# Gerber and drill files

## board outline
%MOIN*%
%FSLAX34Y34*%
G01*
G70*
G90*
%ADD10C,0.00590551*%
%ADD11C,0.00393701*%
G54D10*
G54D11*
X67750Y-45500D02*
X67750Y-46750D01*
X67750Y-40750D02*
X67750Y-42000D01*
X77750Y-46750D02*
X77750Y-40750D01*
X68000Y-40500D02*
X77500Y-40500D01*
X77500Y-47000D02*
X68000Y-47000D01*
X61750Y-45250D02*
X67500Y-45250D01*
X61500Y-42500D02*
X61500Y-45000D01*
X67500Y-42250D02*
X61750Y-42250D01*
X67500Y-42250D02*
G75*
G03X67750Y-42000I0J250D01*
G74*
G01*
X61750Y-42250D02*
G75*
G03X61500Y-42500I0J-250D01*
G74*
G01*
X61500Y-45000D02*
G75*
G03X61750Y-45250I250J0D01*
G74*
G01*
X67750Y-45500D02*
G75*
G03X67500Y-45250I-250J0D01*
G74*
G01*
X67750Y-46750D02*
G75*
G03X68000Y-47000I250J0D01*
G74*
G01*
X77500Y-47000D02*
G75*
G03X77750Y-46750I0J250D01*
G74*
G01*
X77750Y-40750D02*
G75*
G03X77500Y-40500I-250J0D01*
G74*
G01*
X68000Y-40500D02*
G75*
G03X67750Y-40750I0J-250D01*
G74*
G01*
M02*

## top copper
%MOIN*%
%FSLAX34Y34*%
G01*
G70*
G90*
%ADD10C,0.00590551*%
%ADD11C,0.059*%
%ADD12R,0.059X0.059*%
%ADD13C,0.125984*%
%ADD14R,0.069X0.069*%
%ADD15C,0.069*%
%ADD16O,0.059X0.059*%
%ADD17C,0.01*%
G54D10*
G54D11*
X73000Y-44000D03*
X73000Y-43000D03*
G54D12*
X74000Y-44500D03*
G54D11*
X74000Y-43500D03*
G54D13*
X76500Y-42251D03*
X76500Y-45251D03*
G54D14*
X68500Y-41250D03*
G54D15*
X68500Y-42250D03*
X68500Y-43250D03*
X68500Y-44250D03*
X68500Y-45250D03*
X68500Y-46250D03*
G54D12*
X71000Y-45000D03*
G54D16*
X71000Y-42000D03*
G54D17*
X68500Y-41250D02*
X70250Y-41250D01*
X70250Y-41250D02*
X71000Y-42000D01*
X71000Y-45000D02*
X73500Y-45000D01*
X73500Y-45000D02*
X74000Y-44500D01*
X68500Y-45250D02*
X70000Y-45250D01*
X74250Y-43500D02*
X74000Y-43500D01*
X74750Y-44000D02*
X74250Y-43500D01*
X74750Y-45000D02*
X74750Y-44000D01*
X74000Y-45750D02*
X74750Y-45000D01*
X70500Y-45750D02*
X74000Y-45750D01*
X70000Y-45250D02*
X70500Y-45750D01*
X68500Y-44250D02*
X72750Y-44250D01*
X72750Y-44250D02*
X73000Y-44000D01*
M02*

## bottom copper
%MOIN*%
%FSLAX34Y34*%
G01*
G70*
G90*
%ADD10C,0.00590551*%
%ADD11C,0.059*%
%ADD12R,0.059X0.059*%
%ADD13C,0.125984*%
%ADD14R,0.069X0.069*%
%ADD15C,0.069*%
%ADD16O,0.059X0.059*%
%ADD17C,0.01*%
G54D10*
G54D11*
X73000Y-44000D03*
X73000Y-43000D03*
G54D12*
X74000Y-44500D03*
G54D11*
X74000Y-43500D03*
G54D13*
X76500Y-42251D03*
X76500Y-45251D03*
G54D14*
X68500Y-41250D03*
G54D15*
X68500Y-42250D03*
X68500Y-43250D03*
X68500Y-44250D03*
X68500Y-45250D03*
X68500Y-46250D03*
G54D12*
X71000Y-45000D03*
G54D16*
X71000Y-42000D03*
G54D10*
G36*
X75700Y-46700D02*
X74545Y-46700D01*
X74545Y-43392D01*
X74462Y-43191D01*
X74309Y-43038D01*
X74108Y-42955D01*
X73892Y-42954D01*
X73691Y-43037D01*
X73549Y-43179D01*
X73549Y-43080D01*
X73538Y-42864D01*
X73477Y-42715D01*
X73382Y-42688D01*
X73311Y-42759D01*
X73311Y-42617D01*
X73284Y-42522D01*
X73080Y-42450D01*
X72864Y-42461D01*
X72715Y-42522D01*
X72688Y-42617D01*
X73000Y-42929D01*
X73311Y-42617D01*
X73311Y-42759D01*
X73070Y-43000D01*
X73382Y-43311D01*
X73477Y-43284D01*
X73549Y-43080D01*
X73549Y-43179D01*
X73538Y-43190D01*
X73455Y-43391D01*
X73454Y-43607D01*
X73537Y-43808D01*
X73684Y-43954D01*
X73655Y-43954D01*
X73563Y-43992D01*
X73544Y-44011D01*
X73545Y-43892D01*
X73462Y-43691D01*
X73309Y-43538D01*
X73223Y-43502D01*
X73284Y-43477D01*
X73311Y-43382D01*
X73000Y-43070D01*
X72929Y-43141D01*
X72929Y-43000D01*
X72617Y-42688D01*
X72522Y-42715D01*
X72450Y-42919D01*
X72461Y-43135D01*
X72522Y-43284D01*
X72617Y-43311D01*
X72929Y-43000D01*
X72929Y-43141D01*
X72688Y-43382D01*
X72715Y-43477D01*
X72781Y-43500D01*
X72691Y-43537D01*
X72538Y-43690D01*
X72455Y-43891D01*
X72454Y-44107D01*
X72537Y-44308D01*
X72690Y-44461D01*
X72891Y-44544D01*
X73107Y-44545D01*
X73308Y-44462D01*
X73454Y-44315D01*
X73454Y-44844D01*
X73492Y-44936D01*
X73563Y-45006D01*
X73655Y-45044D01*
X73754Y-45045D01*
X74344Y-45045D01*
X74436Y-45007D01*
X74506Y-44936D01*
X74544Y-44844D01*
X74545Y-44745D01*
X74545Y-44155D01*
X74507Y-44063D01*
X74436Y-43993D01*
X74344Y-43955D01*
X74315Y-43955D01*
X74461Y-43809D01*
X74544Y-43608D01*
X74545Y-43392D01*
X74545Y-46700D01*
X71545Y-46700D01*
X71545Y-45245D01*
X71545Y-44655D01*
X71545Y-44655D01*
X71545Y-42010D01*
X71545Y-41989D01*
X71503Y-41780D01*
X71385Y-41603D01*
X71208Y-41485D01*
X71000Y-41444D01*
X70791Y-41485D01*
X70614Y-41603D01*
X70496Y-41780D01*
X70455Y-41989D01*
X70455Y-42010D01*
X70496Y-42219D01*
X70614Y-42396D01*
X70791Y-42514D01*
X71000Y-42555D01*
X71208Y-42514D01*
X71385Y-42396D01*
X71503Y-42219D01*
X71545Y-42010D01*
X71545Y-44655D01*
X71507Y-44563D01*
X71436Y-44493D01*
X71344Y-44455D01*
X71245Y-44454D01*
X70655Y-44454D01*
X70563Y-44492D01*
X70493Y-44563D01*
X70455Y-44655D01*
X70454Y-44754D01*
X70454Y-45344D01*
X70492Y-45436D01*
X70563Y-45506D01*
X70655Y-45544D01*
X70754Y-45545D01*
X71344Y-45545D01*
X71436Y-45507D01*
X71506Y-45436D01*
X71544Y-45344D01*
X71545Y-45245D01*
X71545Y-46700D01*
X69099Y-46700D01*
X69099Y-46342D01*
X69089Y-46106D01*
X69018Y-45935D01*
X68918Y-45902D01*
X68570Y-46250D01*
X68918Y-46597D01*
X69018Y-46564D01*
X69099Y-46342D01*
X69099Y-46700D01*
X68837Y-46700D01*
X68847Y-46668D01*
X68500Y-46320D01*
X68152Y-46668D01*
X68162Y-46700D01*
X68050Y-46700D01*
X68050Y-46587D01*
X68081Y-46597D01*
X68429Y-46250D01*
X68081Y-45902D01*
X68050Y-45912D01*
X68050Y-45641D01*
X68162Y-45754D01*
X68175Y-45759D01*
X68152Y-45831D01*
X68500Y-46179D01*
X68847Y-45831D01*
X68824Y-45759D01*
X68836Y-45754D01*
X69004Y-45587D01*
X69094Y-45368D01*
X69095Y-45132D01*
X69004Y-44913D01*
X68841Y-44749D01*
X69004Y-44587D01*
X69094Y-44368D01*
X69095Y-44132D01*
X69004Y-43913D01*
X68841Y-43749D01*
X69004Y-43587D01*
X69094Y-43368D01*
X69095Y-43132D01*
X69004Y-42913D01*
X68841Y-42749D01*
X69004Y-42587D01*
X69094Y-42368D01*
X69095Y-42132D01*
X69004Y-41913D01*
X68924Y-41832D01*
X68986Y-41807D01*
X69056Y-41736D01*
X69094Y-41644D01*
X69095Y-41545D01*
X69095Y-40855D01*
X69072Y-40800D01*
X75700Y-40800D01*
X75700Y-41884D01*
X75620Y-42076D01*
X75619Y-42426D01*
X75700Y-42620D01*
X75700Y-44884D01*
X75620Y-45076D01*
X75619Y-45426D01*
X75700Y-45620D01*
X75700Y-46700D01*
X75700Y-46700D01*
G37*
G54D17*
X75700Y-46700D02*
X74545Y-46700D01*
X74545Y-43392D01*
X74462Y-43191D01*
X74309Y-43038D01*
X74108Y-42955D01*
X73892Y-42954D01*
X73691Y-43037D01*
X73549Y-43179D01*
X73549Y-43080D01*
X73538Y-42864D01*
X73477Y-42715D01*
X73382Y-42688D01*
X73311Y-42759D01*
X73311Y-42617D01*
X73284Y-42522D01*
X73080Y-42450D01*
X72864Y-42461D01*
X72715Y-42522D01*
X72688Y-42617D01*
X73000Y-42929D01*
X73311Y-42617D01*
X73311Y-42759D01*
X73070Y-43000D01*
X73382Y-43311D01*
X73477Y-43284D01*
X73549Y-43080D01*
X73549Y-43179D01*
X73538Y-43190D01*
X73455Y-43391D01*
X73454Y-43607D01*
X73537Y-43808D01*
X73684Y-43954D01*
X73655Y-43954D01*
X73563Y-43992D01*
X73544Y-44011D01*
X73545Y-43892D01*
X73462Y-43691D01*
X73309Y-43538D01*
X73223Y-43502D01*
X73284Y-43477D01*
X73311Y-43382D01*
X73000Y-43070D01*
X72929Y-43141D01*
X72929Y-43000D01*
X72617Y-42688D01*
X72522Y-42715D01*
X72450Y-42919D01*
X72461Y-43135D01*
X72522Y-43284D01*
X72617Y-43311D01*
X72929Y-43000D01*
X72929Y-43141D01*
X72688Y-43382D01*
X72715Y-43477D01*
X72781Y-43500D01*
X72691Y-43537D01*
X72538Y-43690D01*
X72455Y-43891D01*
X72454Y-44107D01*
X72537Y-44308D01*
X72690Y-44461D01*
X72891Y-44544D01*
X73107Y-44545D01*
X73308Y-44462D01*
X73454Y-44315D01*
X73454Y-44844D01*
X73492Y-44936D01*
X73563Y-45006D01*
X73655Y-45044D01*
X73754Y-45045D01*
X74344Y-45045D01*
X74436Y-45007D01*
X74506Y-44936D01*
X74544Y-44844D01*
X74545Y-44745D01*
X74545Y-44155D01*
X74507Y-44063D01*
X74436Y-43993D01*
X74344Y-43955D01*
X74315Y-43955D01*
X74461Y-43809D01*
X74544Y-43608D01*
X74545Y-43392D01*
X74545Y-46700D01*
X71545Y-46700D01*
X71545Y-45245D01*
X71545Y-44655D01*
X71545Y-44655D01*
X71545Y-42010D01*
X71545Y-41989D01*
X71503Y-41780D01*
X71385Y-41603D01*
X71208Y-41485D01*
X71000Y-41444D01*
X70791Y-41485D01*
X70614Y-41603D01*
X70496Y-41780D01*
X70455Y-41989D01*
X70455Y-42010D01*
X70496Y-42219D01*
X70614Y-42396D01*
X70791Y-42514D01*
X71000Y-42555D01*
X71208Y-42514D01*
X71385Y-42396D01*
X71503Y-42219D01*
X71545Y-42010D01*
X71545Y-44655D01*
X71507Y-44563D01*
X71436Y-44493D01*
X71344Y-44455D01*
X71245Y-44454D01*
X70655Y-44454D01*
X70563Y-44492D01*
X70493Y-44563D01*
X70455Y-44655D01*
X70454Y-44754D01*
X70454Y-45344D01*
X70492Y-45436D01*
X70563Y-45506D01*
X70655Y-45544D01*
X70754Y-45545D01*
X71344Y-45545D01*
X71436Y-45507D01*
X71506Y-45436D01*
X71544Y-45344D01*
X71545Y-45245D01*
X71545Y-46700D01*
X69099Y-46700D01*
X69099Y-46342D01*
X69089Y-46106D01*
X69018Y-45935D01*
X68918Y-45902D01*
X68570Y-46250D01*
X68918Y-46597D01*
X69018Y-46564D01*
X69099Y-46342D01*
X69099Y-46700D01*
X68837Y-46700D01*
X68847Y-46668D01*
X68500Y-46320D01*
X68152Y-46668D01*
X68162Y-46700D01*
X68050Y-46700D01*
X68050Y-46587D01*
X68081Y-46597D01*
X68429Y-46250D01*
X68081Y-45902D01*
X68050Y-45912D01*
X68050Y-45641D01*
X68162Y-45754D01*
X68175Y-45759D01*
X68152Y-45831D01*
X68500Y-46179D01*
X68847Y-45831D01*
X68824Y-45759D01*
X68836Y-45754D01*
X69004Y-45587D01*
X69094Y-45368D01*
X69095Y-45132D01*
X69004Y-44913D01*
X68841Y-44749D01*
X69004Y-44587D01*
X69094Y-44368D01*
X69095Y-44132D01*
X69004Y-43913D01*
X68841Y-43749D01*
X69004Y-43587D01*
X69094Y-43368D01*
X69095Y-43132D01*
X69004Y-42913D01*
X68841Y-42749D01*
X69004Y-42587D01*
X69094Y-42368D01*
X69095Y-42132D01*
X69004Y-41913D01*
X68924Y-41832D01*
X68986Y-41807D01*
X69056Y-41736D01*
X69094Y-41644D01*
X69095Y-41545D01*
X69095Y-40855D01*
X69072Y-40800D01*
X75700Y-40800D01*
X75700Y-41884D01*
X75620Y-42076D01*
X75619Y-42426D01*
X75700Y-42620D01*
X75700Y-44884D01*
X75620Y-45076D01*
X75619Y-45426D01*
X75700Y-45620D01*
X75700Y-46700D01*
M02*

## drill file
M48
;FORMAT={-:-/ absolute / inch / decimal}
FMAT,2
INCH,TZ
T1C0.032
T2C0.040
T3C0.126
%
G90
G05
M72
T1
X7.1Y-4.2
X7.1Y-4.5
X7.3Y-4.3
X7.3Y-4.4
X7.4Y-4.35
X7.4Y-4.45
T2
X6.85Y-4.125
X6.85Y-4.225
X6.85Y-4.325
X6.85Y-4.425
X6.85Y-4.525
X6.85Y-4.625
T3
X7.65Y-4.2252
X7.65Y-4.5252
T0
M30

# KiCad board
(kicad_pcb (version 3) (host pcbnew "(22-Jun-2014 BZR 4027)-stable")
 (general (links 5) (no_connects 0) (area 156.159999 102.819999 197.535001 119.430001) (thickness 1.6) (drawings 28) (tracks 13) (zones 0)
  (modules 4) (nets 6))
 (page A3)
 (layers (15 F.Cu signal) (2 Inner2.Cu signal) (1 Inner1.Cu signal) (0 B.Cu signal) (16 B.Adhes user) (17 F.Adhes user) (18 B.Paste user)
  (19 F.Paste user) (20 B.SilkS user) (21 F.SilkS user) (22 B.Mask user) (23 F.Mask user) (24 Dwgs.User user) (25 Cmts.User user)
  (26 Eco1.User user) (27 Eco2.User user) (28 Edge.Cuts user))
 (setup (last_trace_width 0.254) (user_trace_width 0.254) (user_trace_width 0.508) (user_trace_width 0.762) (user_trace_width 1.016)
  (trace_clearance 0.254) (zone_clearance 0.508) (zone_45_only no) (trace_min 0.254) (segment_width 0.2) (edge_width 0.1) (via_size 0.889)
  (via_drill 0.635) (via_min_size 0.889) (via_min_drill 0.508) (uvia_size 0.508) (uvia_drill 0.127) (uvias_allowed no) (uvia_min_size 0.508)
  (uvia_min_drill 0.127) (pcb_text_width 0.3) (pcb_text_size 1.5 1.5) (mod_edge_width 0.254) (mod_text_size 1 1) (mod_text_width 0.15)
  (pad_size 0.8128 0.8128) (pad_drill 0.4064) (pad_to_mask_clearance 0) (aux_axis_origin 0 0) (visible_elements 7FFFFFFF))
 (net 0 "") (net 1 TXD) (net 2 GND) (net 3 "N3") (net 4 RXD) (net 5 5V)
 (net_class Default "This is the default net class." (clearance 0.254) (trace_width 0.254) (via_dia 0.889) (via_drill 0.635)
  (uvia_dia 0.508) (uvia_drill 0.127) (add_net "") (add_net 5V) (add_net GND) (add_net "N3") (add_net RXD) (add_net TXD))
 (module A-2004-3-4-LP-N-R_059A (layer F.Cu) (at 187.96 113.03 90)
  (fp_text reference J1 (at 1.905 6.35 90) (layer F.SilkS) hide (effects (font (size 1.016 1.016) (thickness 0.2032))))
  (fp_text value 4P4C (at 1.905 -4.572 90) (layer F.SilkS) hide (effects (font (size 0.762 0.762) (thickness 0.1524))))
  (pad 2 thru_hole circle (at 1.27 -2.54 90) (size 1.4986 1.4986) (drill 0.8128) (layers *.Cu *.Mask F.SilkS) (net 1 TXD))
  (pad 4 thru_hole circle (at 3.81 -2.54 90) (size 1.4986 1.4986) (drill 0.8128) (layers *.Cu *.Mask F.SilkS) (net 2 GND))
  (pad 1 thru_hole rect (at 0 0 90) (size 1.4986 1.4986) (drill 0.8128) (layers *.Cu *.Mask F.SilkS) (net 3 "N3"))
  (pad 3 thru_hole circle (at 2.54 0 90) (size 1.4986 1.4986) (drill 0.8128) (layers *.Cu *.Mask F.SilkS) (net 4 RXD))
  (pad "" thru_hole circle (at 5.71 6.35 90) (size 3.2 3.2) (drill 3.2) (layers *.Cu *.Mask F.SilkS))
  (pad "" thru_hole circle (at -1.91 6.35 90) (size 3.2 3.2) (drill 3.2) (layers *.Cu *.Mask F.SilkS)))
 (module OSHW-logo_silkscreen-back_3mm (layer F.Cu) (at 169.545 111.125)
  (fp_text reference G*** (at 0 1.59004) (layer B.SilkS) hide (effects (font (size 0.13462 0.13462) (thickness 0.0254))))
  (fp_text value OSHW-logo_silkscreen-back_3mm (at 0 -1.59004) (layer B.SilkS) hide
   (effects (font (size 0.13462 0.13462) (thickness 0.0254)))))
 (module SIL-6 (layer F.Cu) (at 173.99 107.315 270)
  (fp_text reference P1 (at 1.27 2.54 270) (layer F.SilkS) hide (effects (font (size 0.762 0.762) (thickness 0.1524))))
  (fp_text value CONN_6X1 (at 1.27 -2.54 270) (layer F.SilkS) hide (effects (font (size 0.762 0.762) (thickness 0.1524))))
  (pad 1 thru_hole rect (at -2.54 0 270) (size 1.7526 1.7526) (drill 1.016) (layers *.Cu *.Mask F.SilkS) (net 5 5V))
  (pad 2 thru_hole circle (at 0 0 270) (size 1.7526 1.7526) (drill 1.016) (layers *.Cu *.Mask F.SilkS))
  (pad 3 thru_hole circle (at 2.54 0 270) (size 1.7526 1.7526) (drill 1.016) (layers *.Cu *.Mask F.SilkS))
  (pad 4 thru_hole circle (at 5.08 0 270) (size 1.7526 1.7526) (drill 1.016) (layers *.Cu *.Mask F.SilkS) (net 1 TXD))
  (pad 5 thru_hole circle (at 7.62 0 270) (size 1.7526 1.7526) (drill 1.016) (layers *.Cu *.Mask F.SilkS) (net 4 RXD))
  (pad 6 thru_hole circle (at 10.16 0 270) (size 1.7526 1.7526) (drill 1.016) (layers *.Cu *.Mask F.SilkS) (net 2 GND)))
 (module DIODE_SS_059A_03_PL (layer F.Cu) (at 180.34 110.49 270)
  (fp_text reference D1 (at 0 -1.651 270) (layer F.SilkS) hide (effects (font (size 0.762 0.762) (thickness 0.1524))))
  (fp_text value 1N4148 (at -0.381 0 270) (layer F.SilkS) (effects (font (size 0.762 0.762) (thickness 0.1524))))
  (pad 2 thru_hole rect (at 3.81 0 270) (size 1.4986 1.4986) (drill 0.8128) (layers *.Cu *.Mask F.SilkS) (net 3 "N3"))
  (pad 1 thru_hole oval (at -3.81 0 270) (size 1.4986 1.4986) (drill 0.8128) (layers *.Cu *.Mask F.SilkS) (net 5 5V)))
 (gr_line (start 172.085 115.57) (end 172.085 118.745) (angle 90) (layer Edge.Cuts) (width 0.1))
 (gr_line (start 172.085 103.505) (end 172.085 106.68) (angle 90) (layer Edge.Cuts) (width 0.1))
 (gr_line (start 197.485 118.745) (end 197.485 103.505) (angle 90) (layer Edge.Cuts) (width 0.1))
 (gr_line (start 172.72 102.87) (end 196.85 102.87) (angle 90) (layer Edge.Cuts) (width 0.1))
 (gr_line (start 196.85 119.38) (end 172.72 119.38) (angle 90) (layer Edge.Cuts) (width 0.1))
 (gr_line (start 156.845 114.935) (end 171.45 114.935) (angle 90) (layer Edge.Cuts) (width 0.1))
 (gr_line (start 156.21 107.95) (end 156.21 114.3) (angle 90) (layer Edge.Cuts) (width 0.1))
 (gr_line (start 171.45 107.315) (end 156.845 107.315) (angle 90) (layer Edge.Cuts) (width 0.1))
 (gr_arc (start 171.45 106.68) (end 172.085 106.68) (angle 90) (layer Edge.Cuts) (width 0.1))
 (gr_arc (start 156.845 107.95) (end 156.21 107.95) (angle 90) (layer Edge.Cuts) (width 0.1))
 (gr_arc (start 156.845 114.3) (end 156.845 114.935) (angle 90) (layer Edge.Cuts) (width 0.1))
 (gr_arc (start 171.45 115.57) (end 171.45 114.935) (angle 90) (layer Edge.Cuts) (width 0.1))
 (gr_arc (start 172.72 118.745) (end 172.72 119.38) (angle 90) (layer Edge.Cuts) (width 0.1))
 (gr_arc (start 196.85 118.745) (end 197.485 118.745) (angle 90) (layer Edge.Cuts) (width 0.1))
 (gr_arc (start 196.85 103.505) (end 196.85 102.87) (angle 90) (layer Edge.Cuts) (width 0.1))
 (gr_arc (start 172.72 103.505) (end 172.085 103.505) (angle 90) (layer Edge.Cuts) (width 0.1))
 (segment (start 173.99 104.775) (end 178.435 104.775) (width 0.254) (layer F.Cu) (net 5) (status 400000))
 (segment (start 178.435 104.775) (end 180.34 106.68) (width 0.254) (layer F.Cu) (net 5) (status 800000))
 (segment (start 180.34 114.3) (end 186.69 114.3) (width 0.254) (layer F.Cu) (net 3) (status 400000))
 (segment (start 186.69 114.3) (end 187.96 113.03) (width 0.254) (layer F.Cu) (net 3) (status 800000))
 (segment (start 173.99 114.935) (end 177.8 114.935) (width 0.254) (layer F.Cu) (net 4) (status 400000))
 (segment (start 188.595 110.49) (end 187.96 110.49) (width 0.254) (layer F.Cu) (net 4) (status C00000))
 (segment (start 189.865 111.76) (end 188.595 110.49) (width 0.254) (layer F.Cu) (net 4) (status 800000))
 (segment (start 189.865 114.3) (end 189.865 111.76) (width 0.254) (layer F.Cu) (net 4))
 (segment (start 187.96 116.205) (end 189.865 114.3) (width 0.254) (layer F.Cu) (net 4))
 (segment (start 179.07 116.205) (end 187.96 116.205) (width 0.254) (layer F.Cu) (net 4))
 (segment (start 177.8 114.935) (end 179.07 116.205) (width 0.254) (layer F.Cu) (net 4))
 (segment (start 173.99 112.395) (end 184.785 112.395) (width 0.254) (layer F.Cu) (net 1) (status 400000))
 (segment (start 184.785 112.395) (end 185.42 111.76) (width 0.254) (layer F.Cu) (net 1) (status 800000))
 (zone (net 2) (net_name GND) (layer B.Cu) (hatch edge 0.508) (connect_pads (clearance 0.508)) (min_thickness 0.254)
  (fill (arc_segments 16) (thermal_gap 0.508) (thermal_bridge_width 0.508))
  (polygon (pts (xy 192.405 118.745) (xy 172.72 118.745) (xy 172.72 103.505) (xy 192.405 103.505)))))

